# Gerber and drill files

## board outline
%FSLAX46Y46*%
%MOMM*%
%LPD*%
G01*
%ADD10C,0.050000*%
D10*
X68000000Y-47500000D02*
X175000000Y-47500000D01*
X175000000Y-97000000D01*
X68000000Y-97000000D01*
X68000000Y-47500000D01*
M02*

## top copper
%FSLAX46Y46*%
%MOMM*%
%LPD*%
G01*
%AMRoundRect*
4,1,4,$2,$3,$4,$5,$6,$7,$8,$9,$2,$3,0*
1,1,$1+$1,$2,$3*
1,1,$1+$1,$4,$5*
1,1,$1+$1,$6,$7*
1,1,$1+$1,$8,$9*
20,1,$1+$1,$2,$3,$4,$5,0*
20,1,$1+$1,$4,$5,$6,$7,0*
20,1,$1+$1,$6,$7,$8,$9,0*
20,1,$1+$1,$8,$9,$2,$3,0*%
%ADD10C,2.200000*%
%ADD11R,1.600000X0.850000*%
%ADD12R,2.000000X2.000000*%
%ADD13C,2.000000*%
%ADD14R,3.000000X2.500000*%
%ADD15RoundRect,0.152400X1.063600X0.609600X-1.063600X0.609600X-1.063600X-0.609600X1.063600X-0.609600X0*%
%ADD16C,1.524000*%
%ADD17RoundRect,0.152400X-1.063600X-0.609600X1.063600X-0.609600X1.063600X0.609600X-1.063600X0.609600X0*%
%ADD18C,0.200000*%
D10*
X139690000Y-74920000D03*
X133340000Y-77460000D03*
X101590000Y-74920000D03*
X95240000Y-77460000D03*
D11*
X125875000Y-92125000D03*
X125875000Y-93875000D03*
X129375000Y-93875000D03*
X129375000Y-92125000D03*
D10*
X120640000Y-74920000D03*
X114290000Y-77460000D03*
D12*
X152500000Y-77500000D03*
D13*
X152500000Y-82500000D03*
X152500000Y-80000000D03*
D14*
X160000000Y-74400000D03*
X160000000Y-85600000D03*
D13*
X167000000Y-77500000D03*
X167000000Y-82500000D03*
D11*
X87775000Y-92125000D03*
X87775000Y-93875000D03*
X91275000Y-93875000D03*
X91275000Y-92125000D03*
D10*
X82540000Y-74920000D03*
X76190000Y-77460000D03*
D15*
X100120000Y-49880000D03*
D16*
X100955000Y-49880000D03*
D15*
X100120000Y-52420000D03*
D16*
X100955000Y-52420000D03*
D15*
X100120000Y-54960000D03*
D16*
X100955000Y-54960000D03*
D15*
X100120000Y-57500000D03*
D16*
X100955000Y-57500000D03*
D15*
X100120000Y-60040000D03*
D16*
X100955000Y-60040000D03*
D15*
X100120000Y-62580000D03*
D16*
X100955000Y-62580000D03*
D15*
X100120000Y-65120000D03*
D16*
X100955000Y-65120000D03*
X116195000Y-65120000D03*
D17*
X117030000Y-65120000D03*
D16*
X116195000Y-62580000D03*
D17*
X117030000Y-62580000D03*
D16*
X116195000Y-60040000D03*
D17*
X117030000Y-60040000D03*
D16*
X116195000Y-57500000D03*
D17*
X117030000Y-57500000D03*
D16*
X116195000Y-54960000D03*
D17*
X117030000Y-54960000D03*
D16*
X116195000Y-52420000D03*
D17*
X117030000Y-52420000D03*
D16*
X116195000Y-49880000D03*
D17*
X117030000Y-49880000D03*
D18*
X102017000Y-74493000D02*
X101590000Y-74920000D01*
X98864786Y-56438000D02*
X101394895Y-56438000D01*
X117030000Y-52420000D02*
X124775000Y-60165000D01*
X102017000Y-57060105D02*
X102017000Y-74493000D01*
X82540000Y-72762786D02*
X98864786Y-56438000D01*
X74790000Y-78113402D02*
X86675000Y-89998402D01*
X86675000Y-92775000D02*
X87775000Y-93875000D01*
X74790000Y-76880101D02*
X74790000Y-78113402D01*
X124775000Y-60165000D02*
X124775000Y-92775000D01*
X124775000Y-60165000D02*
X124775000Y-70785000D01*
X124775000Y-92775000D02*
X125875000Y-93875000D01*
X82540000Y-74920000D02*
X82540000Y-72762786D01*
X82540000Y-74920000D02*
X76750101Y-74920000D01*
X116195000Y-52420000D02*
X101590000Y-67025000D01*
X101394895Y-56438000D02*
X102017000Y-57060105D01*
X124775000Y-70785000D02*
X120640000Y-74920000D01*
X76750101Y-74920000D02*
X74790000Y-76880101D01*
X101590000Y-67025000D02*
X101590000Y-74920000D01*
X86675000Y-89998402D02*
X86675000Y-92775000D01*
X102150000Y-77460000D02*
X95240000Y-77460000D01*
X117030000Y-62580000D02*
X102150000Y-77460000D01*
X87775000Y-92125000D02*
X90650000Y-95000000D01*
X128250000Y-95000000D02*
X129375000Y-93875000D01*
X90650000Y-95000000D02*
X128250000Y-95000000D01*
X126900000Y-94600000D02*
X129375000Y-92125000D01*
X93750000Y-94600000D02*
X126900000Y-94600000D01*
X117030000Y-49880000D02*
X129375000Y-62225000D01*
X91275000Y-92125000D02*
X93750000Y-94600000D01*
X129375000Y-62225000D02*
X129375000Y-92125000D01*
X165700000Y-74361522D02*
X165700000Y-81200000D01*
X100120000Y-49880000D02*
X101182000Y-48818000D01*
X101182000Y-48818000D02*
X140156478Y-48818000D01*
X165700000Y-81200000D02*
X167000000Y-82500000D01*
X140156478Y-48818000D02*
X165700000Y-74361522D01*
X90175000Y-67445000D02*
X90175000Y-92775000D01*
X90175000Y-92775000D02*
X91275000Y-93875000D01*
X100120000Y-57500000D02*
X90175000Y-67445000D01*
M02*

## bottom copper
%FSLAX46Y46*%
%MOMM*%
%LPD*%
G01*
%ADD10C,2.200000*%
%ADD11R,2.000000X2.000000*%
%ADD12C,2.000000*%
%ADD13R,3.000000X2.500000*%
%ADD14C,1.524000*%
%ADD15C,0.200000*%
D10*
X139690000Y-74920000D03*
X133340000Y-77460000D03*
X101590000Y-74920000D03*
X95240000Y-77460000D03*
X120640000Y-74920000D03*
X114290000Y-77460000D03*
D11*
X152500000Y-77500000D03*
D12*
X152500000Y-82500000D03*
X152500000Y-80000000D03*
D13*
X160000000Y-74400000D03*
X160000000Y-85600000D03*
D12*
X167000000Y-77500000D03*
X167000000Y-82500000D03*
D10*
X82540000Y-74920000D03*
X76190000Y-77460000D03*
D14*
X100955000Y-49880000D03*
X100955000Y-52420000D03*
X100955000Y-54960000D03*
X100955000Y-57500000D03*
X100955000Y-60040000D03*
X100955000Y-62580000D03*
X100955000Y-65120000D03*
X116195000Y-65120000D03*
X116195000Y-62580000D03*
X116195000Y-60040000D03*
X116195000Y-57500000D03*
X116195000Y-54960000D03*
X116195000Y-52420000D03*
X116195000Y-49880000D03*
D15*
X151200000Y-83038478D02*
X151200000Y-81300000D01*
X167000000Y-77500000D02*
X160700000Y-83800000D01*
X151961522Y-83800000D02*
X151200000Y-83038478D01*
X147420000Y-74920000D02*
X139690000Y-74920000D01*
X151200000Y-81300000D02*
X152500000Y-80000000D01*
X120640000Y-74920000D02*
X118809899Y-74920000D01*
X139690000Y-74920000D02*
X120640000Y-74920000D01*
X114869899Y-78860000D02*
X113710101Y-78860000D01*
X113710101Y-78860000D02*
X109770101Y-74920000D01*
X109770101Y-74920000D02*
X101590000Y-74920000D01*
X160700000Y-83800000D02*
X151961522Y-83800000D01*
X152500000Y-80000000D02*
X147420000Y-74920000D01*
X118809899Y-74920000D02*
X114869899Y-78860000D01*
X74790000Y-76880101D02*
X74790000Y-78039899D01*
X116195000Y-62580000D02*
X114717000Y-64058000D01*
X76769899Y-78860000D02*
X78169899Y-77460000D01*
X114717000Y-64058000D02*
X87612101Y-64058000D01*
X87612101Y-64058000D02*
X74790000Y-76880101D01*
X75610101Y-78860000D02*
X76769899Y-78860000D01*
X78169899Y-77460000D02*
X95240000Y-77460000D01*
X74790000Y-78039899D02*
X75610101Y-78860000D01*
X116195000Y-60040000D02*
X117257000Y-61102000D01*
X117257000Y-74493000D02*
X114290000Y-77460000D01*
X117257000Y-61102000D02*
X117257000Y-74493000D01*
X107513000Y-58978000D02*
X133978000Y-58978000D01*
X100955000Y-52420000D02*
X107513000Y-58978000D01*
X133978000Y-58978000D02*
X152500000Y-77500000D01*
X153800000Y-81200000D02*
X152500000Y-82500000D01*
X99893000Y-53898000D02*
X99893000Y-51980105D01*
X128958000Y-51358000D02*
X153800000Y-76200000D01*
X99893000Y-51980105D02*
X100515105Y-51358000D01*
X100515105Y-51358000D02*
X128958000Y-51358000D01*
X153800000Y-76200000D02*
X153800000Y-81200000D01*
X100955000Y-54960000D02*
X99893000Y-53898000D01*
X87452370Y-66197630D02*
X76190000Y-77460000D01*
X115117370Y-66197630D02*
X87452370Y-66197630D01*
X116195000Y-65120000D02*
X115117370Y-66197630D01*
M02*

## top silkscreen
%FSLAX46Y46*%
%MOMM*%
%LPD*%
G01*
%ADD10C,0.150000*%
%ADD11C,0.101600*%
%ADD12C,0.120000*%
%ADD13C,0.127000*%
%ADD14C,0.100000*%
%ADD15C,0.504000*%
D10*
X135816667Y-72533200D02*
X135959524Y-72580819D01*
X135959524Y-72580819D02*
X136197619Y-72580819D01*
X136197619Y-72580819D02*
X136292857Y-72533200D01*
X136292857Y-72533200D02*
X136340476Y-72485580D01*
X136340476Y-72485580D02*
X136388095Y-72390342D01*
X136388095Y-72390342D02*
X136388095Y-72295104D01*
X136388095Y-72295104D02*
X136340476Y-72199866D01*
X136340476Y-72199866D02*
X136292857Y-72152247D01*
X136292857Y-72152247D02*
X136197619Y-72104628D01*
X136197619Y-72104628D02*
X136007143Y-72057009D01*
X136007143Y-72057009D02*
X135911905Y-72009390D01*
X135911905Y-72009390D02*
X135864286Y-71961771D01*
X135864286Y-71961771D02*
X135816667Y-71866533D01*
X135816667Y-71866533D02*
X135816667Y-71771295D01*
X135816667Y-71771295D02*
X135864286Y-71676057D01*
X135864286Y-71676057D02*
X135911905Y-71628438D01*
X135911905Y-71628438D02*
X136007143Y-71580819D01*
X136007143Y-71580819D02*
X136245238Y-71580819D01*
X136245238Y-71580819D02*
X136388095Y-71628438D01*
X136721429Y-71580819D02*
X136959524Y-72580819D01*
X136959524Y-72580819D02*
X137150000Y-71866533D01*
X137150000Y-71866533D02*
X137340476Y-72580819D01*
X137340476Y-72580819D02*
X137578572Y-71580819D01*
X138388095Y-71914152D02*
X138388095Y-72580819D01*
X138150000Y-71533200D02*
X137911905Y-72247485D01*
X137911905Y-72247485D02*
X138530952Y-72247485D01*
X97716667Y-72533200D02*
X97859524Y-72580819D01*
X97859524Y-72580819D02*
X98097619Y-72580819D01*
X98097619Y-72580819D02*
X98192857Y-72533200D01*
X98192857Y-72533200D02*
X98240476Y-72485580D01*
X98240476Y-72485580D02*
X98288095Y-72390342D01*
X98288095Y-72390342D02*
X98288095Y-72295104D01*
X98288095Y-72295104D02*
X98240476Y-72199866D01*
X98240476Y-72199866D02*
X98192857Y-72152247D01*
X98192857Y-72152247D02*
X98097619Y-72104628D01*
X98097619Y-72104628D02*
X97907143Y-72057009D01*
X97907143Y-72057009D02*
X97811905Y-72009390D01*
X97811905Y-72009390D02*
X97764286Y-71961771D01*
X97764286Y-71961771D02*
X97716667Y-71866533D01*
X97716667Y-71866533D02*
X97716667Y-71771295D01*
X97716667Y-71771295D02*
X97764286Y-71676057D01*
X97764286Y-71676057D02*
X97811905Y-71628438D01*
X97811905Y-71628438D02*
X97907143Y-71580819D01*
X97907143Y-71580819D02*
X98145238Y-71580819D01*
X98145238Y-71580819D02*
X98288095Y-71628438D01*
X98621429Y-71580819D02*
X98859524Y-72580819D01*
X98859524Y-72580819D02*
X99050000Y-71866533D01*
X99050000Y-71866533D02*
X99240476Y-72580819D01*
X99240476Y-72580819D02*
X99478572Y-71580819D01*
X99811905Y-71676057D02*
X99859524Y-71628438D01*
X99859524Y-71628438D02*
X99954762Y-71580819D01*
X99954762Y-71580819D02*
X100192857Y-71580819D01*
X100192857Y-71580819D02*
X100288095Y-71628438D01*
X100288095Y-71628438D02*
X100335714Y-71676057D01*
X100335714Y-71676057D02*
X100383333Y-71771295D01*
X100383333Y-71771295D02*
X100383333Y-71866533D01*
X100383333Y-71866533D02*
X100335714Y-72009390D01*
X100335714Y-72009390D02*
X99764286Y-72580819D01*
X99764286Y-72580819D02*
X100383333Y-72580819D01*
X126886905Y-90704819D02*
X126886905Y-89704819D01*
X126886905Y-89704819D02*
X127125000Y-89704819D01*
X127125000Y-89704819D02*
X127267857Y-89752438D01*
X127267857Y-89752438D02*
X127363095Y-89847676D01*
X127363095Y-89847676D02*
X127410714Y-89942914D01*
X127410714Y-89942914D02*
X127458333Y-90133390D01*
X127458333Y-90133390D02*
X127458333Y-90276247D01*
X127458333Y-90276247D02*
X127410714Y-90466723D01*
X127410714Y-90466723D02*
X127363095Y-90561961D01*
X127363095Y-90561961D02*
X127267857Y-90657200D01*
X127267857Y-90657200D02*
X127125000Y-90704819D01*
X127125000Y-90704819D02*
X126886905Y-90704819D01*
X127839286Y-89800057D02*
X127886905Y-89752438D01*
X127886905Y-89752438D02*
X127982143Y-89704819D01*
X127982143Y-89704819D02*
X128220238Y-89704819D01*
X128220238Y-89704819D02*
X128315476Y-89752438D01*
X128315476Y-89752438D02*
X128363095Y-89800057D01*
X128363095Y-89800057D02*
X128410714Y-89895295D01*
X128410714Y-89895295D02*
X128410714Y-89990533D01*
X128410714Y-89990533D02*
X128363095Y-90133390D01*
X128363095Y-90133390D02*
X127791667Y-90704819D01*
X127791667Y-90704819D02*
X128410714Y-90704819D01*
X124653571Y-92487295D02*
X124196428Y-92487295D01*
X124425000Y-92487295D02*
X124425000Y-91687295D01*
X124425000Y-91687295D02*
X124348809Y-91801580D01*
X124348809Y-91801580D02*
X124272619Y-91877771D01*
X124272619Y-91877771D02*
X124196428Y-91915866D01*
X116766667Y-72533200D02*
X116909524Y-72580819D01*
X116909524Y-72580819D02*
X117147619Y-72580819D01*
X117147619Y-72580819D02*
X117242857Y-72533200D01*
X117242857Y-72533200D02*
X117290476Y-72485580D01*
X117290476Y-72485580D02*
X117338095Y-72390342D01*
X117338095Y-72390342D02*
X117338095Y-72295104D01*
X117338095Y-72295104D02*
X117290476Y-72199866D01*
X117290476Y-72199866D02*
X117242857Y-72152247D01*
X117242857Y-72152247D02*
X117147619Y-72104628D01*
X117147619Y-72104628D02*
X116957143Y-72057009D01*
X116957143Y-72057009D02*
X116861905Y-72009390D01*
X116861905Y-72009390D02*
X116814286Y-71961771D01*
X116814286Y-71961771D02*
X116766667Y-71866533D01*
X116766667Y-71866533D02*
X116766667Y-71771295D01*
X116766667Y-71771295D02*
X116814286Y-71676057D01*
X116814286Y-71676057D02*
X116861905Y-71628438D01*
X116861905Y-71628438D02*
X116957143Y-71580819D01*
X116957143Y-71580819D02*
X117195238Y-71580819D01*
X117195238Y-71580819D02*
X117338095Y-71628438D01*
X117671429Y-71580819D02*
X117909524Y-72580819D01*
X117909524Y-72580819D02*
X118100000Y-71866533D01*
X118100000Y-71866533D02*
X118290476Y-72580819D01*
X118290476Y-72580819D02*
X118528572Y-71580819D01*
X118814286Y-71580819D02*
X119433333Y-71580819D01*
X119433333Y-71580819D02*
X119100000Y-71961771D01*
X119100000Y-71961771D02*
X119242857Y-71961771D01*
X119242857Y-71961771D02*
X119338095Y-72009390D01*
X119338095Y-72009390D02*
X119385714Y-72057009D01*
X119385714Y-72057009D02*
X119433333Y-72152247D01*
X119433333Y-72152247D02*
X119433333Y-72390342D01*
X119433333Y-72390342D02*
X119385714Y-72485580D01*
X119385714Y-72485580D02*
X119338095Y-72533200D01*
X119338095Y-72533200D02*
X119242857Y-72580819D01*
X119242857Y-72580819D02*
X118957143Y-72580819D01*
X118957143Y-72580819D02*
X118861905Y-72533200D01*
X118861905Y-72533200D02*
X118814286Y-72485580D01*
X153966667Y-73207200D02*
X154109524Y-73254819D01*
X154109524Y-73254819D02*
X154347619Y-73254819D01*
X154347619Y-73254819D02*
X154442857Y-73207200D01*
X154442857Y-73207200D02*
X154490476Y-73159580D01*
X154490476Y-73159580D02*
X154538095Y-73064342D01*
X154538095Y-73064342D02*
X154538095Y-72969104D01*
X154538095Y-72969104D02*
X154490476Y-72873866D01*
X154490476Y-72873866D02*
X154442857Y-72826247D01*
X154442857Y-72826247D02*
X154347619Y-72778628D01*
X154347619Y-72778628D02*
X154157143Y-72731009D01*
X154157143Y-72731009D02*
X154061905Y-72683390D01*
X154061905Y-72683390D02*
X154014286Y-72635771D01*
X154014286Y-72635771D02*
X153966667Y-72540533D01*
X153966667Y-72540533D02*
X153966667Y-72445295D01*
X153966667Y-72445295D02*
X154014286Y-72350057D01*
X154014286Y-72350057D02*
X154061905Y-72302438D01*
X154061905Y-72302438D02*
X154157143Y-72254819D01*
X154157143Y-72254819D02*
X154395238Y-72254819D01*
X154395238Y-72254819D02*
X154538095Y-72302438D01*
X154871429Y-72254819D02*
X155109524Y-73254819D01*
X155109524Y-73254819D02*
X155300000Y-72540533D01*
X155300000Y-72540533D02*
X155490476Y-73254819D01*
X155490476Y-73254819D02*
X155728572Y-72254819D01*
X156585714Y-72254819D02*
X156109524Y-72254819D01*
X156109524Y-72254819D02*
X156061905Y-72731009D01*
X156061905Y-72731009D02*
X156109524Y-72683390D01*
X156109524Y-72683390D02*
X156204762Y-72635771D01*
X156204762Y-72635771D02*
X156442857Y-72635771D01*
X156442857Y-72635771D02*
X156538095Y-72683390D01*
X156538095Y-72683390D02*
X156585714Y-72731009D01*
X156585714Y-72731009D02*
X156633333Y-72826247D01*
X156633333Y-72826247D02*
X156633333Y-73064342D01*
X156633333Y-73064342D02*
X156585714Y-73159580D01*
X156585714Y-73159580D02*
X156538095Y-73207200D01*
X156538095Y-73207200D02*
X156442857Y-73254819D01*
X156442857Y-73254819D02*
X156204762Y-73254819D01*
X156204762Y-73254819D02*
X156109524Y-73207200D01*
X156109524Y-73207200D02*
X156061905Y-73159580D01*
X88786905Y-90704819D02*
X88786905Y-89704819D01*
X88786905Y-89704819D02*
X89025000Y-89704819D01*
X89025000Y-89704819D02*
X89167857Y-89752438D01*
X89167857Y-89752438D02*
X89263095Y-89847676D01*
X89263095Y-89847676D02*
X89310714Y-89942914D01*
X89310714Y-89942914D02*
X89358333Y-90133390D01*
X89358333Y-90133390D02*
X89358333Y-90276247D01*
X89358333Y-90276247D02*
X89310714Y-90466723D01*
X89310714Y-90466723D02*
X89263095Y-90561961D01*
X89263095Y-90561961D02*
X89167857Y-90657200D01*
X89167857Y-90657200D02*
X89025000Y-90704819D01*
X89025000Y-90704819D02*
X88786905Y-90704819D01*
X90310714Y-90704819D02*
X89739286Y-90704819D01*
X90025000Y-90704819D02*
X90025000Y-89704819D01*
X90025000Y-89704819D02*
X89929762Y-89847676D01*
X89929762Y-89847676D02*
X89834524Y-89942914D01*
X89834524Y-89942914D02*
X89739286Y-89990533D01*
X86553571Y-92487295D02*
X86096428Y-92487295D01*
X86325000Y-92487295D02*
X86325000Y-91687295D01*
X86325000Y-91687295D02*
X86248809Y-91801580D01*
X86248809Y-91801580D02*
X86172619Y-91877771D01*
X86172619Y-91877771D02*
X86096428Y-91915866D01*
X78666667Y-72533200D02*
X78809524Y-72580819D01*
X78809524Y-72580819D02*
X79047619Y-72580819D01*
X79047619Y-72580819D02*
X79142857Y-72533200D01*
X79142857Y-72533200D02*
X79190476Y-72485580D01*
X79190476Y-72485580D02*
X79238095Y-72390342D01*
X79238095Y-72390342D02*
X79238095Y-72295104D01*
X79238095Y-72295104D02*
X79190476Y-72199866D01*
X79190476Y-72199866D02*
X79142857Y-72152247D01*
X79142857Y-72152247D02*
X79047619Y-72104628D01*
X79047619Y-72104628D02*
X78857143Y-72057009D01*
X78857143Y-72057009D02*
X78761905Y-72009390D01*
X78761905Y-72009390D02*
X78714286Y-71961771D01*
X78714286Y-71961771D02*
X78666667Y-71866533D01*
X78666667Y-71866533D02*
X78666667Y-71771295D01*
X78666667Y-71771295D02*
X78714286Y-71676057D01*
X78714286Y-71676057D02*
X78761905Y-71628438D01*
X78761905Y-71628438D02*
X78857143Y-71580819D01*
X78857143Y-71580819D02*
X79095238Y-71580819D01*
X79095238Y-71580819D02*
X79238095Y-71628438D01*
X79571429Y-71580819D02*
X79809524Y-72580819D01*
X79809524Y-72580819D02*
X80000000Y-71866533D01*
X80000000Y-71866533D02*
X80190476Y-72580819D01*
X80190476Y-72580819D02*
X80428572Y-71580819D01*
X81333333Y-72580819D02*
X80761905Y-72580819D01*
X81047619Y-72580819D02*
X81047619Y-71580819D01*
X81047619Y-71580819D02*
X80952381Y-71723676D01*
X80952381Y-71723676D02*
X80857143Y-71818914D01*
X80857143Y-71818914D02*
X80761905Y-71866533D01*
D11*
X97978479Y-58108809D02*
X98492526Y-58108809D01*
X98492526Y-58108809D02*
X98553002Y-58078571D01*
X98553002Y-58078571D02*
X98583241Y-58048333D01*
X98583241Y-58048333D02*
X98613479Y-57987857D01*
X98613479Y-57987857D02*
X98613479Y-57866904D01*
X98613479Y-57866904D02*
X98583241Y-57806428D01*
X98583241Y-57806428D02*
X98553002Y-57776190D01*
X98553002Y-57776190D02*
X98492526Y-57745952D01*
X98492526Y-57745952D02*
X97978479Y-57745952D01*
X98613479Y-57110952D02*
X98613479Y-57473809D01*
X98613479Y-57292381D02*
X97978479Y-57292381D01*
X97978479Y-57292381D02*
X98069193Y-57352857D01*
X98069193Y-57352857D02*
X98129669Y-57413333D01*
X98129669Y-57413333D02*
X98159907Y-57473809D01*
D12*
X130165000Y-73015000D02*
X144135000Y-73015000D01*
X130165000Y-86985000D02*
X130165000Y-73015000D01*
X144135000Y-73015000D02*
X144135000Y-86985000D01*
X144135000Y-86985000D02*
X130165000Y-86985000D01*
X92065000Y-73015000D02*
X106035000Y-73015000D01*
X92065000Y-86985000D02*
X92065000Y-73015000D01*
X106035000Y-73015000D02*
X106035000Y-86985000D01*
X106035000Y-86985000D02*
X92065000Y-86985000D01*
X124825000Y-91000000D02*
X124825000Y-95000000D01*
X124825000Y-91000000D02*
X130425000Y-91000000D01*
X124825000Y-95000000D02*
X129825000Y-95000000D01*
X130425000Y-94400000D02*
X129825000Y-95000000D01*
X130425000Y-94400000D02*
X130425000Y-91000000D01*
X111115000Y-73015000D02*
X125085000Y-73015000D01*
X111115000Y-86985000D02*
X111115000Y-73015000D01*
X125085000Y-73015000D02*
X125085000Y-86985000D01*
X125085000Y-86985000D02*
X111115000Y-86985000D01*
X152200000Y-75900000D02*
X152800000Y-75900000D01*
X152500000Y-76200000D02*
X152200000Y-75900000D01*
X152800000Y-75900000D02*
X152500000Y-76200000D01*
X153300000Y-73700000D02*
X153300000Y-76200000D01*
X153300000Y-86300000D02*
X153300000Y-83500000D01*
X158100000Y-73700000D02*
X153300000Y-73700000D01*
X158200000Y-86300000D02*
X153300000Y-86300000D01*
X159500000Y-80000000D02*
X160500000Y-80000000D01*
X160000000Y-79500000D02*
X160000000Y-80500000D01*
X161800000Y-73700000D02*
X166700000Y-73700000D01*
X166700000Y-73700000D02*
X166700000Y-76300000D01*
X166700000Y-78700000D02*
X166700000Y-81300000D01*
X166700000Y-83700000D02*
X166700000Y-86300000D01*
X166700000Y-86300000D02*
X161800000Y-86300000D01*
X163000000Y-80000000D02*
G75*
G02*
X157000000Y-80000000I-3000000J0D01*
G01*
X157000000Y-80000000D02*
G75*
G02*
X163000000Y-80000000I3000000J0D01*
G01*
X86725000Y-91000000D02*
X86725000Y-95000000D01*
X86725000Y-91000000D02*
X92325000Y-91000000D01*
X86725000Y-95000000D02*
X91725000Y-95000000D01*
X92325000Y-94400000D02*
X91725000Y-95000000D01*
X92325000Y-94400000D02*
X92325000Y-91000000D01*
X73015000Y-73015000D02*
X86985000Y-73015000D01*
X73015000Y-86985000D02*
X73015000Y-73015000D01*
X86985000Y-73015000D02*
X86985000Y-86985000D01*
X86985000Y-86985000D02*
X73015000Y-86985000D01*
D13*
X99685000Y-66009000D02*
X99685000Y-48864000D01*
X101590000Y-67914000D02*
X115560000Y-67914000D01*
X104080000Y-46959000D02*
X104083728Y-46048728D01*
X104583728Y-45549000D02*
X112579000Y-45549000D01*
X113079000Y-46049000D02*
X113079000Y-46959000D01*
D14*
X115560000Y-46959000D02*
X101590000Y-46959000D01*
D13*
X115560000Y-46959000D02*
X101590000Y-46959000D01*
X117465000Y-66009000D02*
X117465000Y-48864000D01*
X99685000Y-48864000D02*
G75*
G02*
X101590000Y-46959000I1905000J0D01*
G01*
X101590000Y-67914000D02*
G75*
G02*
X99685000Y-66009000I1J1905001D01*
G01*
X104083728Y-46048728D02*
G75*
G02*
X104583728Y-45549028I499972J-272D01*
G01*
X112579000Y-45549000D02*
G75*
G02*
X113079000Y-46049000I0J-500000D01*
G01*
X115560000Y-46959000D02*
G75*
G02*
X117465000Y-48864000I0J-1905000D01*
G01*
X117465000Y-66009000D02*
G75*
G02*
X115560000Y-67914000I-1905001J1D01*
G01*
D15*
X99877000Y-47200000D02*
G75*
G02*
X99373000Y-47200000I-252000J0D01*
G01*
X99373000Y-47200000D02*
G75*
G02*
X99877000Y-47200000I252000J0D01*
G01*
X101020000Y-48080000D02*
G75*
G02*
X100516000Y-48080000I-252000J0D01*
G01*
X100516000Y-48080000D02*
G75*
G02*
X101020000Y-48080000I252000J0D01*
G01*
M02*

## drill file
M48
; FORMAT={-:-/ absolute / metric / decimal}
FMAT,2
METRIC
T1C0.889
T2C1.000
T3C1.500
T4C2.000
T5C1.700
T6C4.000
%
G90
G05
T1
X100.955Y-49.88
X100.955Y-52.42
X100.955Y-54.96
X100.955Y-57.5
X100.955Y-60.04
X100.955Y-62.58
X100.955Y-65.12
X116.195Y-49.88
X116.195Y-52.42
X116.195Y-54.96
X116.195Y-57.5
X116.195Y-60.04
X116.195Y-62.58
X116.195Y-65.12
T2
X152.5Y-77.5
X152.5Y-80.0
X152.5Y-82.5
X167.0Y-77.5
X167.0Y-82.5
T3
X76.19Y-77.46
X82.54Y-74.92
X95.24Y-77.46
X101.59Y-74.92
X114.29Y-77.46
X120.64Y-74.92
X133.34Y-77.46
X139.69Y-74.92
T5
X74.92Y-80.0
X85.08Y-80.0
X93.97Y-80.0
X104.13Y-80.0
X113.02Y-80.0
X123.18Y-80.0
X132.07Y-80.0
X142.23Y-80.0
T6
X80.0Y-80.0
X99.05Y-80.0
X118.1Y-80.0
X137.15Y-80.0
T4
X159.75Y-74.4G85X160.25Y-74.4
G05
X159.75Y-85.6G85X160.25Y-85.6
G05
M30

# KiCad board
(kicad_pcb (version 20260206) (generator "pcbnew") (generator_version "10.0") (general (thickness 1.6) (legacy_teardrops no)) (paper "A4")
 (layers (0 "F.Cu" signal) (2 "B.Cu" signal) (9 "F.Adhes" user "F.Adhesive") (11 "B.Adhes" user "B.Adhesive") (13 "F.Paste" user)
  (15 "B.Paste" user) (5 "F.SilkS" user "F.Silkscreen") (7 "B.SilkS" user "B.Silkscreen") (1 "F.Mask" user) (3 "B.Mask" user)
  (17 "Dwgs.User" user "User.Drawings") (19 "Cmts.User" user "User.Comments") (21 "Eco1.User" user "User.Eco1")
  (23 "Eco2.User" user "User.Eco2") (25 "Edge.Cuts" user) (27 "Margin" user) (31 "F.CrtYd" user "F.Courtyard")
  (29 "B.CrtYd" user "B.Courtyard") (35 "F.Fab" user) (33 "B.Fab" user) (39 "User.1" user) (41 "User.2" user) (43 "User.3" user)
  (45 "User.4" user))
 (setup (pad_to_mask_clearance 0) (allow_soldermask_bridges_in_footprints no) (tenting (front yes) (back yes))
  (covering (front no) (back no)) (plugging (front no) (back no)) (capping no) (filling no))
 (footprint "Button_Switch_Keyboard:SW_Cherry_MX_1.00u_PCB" (layer "F.Cu") (at 139.69 74.92)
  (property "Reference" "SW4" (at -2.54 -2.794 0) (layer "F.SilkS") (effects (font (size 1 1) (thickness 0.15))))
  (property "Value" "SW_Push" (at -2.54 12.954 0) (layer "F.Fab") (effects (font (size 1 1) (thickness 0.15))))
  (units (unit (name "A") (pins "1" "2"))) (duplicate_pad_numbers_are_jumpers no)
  (fp_line (start -9.525 -1.905) (end 4.445 -1.905) (stroke (width 0.12) (type solid)) (layer "F.SilkS"))
  (fp_line (start -9.525 12.065) (end -9.525 -1.905) (stroke (width 0.12) (type solid)) (layer "F.SilkS"))
  (fp_line (start 4.445 -1.905) (end 4.445 12.065) (stroke (width 0.12) (type solid)) (layer "F.SilkS"))
  (fp_line (start 4.445 12.065) (end -9.525 12.065) (stroke (width 0.12) (type solid)) (layer "F.SilkS"))
  (pad "" np_thru_hole circle (at -7.62 5.08) (size 1.7 1.7) (drill 1.7) (layers "*.Cu" "*.Mask"))
  (pad "" np_thru_hole circle (at -2.54 5.08) (size 4 4) (drill 4) (layers "*.Cu" "*.Mask"))
  (pad "" np_thru_hole circle (at 2.54 5.08) (size 1.7 1.7) (drill 1.7) (layers "*.Cu" "*.Mask"))
  (pad "1" thru_hole circle (at 0 0) (size 2.2 2.2) (drill 1.5) (layers "*.Cu" "*.Mask") (remove_unused_layers no) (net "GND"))
  (pad "2" thru_hole circle (at -6.35 2.54) (size 2.2 2.2) (drill 1.5) (layers "*.Cu" "*.Mask") (remove_unused_layers no)
   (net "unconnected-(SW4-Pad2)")))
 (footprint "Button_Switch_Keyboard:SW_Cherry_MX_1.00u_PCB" (layer "F.Cu") (at 101.59 74.92)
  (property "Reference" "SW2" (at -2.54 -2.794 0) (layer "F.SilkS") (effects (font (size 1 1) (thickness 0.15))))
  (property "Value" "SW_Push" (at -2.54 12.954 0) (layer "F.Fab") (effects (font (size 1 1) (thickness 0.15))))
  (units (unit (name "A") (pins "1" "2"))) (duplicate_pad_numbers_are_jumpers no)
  (fp_line (start -9.525 -1.905) (end 4.445 -1.905) (stroke (width 0.12) (type solid)) (layer "F.SilkS"))
  (fp_line (start -9.525 12.065) (end -9.525 -1.905) (stroke (width 0.12) (type solid)) (layer "F.SilkS"))
  (fp_line (start 4.445 -1.905) (end 4.445 12.065) (stroke (width 0.12) (type solid)) (layer "F.SilkS"))
  (fp_line (start 4.445 12.065) (end -9.525 12.065) (stroke (width 0.12) (type solid)) (layer "F.SilkS"))
  (pad "" np_thru_hole circle (at -7.62 5.08) (size 1.7 1.7) (drill 1.7) (layers "*.Cu" "*.Mask"))
  (pad "" np_thru_hole circle (at -2.54 5.08) (size 4 4) (drill 4) (layers "*.Cu" "*.Mask"))
  (pad "" np_thru_hole circle (at 2.54 5.08) (size 1.7 1.7) (drill 1.7) (layers "*.Cu" "*.Mask"))
  (pad "1" thru_hole circle (at 0 0) (size 2.2 2.2) (drill 1.5) (layers "*.Cu" "*.Mask") (remove_unused_layers no) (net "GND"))
  (pad "2" thru_hole circle (at -6.35 2.54) (size 2.2 2.2) (drill 1.5) (layers "*.Cu" "*.Mask") (remove_unused_layers no)
   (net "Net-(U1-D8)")))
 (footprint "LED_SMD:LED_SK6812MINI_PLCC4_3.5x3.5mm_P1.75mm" (layer "F.Cu") (at 127.625 93)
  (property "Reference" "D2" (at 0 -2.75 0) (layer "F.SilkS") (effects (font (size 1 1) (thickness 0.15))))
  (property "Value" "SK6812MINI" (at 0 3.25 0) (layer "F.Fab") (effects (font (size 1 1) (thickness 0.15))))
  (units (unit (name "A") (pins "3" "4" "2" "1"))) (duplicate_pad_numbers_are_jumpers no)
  (fp_line (start -2.8 -2) (end -2.8 2) (stroke (width 0.12) (type default)) (layer "F.SilkS"))
  (fp_line (start -2.8 -2) (end 2.8 -2) (stroke (width 0.12) (type solid)) (layer "F.SilkS"))
  (fp_line (start -2.8 2) (end 2.2 2) (stroke (width 0.12) (type solid)) (layer "F.SilkS"))
  (fp_line (start 2.8 1.4) (end 2.2 2) (stroke (width 0.12) (type default)) (layer "F.SilkS"))
  (fp_line (start 2.8 1.4) (end 2.8 -2) (stroke (width 0.12) (type solid)) (layer "F.SilkS"))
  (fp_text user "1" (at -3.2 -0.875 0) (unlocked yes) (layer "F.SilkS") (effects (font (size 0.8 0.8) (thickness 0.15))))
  (pad "1" smd rect (at -1.75 -0.875) (size 1.6 0.85) (layers "F.Cu" "F.Mask" "F.Paste") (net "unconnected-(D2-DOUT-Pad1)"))
  (pad "2" smd rect (at -1.75 0.875) (size 1.6 0.85) (layers "F.Cu" "F.Mask" "F.Paste") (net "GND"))
  (pad "3" smd rect (at 1.75 0.875) (size 1.6 0.85) (layers "F.Cu" "F.Mask" "F.Paste") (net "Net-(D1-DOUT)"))
  (pad "4" smd rect (at 1.75 -0.875) (size 1.6 0.85) (layers "F.Cu" "F.Mask" "F.Paste") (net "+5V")))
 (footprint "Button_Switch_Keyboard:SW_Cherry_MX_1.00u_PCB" (layer "F.Cu") (at 120.64 74.92)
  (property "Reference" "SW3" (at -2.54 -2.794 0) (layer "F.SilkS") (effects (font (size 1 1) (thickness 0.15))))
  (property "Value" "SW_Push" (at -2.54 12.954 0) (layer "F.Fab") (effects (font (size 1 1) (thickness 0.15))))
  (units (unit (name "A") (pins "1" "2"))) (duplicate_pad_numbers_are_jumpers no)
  (fp_line (start -9.525 -1.905) (end 4.445 -1.905) (stroke (width 0.12) (type solid)) (layer "F.SilkS"))
  (fp_line (start -9.525 12.065) (end -9.525 -1.905) (stroke (width 0.12) (type solid)) (layer "F.SilkS"))
  (fp_line (start 4.445 -1.905) (end 4.445 12.065) (stroke (width 0.12) (type solid)) (layer "F.SilkS"))
  (fp_line (start 4.445 12.065) (end -9.525 12.065) (stroke (width 0.12) (type solid)) (layer "F.SilkS"))
  (pad "" np_thru_hole circle (at -7.62 5.08) (size 1.7 1.7) (drill 1.7) (layers "*.Cu" "*.Mask"))
  (pad "" np_thru_hole circle (at -2.54 5.08) (size 4 4) (drill 4) (layers "*.Cu" "*.Mask"))
  (pad "" np_thru_hole circle (at 2.54 5.08) (size 1.7 1.7) (drill 1.7) (layers "*.Cu" "*.Mask"))
  (pad "1" thru_hole circle (at 0 0) (size 2.2 2.2) (drill 1.5) (layers "*.Cu" "*.Mask") (remove_unused_layers no) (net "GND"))
  (pad "2" thru_hole circle (at -6.35 2.54) (size 2.2 2.2) (drill 1.5) (layers "*.Cu" "*.Mask") (remove_unused_layers no)
   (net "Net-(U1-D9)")))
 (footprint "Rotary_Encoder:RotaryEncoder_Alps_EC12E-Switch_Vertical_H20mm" (layer "F.Cu") (at 152.5 77.5)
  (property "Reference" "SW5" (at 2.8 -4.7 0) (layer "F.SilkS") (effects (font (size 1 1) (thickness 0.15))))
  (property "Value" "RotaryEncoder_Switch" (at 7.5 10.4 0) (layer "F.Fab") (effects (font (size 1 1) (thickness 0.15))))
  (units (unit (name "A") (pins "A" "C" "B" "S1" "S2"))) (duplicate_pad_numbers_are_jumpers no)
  (fp_line (start -0.3 -1.6) (end 0.3 -1.6) (stroke (width 0.12) (type solid)) (layer "F.SilkS"))
  (fp_line (start 0 -1.3) (end -0.3 -1.6) (stroke (width 0.12) (type solid)) (layer "F.SilkS"))
  (fp_line (start 0.3 -1.6) (end 0 -1.3) (stroke (width 0.12) (type solid)) (layer "F.SilkS"))
  (fp_line (start 0.8 -3.8) (end 0.8 -1.3) (stroke (width 0.12) (type solid)) (layer "F.SilkS"))
  (fp_line (start 0.8 8.8) (end 0.8 6) (stroke (width 0.12) (type solid)) (layer "F.SilkS"))
  (fp_line (start 5.6 -3.8) (end 0.8 -3.8) (stroke (width 0.12) (type solid)) (layer "F.SilkS"))
  (fp_line (start 5.7 8.8) (end 0.8 8.8) (stroke (width 0.12) (type solid)) (layer "F.SilkS"))
  (fp_line (start 7 2.5) (end 8 2.5) (stroke (width 0.12) (type solid)) (layer "F.SilkS"))
  (fp_line (start 7.5 2) (end 7.5 3) (stroke (width 0.12) (type solid)) (layer "F.SilkS"))
  (fp_line (start 9.3 -3.8) (end 14.2 -3.8) (stroke (width 0.12) (type solid)) (layer "F.SilkS"))
  (fp_line (start 14.2 -3.8) (end 14.2 -1.2) (stroke (width 0.12) (type solid)) (layer "F.SilkS"))
  (fp_line (start 14.2 1.2) (end 14.2 3.8) (stroke (width 0.12) (type solid)) (layer "F.SilkS"))
  (fp_line (start 14.2 6.2) (end 14.2 8.8) (stroke (width 0.12) (type solid)) (layer "F.SilkS"))
  (fp_line (start 14.2 8.8) (end 9.3 8.8) (stroke (width 0.12) (type solid)) (layer "F.SilkS"))
  (fp_circle (center 7.5 2.5) (end 10.5 2.5) (stroke (width 0.12) (type solid)) (fill no) (layer "F.SilkS"))
  (pad "A" thru_hole rect (at 0 0) (size 2 2) (drill 1) (layers "*.Cu" "*.Mask") (remove_unused_layers no) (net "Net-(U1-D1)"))
  (pad "B" thru_hole circle (at 0 5) (size 2 2) (drill 1) (layers "*.Cu" "*.Mask") (remove_unused_layers no) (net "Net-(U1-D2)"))
  (pad "C" thru_hole circle (at 0 2.5) (size 2 2) (drill 1) (layers "*.Cu" "*.Mask") (remove_unused_layers no) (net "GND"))
  (pad "MP" thru_hole rect (at 7.5 -3.1) (size 3 2.5) (drill oval 2.5 2) (layers "*.Cu" "*.Mask") (remove_unused_layers no))
  (pad "MP" thru_hole rect (at 7.5 8.1) (size 3 2.5) (drill oval 2.5 2) (layers "*.Cu" "*.Mask") (remove_unused_layers no))
  (pad "S1" thru_hole circle (at 14.5 0) (size 2 2) (drill 1) (layers "*.Cu" "*.Mask") (remove_unused_layers no) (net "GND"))
  (pad "S2" thru_hole circle (at 14.5 5) (size 2 2) (drill 1) (layers "*.Cu" "*.Mask") (remove_unused_layers no) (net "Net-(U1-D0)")))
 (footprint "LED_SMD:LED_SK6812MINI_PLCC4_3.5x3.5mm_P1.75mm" (layer "F.Cu") (at 89.525 93)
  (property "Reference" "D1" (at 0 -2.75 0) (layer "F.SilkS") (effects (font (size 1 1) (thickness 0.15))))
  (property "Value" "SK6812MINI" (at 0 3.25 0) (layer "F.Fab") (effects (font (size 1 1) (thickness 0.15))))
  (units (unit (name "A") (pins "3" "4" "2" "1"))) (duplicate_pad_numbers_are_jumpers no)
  (fp_line (start -2.8 -2) (end -2.8 2) (stroke (width 0.12) (type default)) (layer "F.SilkS"))
  (fp_line (start -2.8 -2) (end 2.8 -2) (stroke (width 0.12) (type solid)) (layer "F.SilkS"))
  (fp_line (start -2.8 2) (end 2.2 2) (stroke (width 0.12) (type solid)) (layer "F.SilkS"))
  (fp_line (start 2.8 1.4) (end 2.2 2) (stroke (width 0.12) (type default)) (layer "F.SilkS"))
  (fp_line (start 2.8 1.4) (end 2.8 -2) (stroke (width 0.12) (type solid)) (layer "F.SilkS"))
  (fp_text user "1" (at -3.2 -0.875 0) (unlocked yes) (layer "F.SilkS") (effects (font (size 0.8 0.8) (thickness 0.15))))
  (pad "1" smd rect (at -1.75 -0.875) (size 1.6 0.85) (layers "F.Cu" "F.Mask" "F.Paste") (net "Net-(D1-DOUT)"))
  (pad "2" smd rect (at -1.75 0.875) (size 1.6 0.85) (layers "F.Cu" "F.Mask" "F.Paste") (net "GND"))
  (pad "3" smd rect (at 1.75 0.875) (size 1.6 0.85) (layers "F.Cu" "F.Mask" "F.Paste") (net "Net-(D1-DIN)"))
  (pad "4" smd rect (at 1.75 -0.875) (size 1.6 0.85) (layers "F.Cu" "F.Mask" "F.Paste") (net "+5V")))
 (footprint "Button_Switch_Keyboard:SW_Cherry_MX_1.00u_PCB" (layer "F.Cu") (at 82.54 74.92)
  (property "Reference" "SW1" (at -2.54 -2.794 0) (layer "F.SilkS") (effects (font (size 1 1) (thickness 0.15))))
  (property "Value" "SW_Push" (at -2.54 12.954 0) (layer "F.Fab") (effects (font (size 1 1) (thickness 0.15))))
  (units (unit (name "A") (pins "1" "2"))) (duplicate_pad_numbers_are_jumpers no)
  (fp_line (start -9.525 -1.905) (end 4.445 -1.905) (stroke (width 0.12) (type solid)) (layer "F.SilkS"))
  (fp_line (start -9.525 12.065) (end -9.525 -1.905) (stroke (width 0.12) (type solid)) (layer "F.SilkS"))
  (fp_line (start 4.445 -1.905) (end 4.445 12.065) (stroke (width 0.12) (type solid)) (layer "F.SilkS"))
  (fp_line (start 4.445 12.065) (end -9.525 12.065) (stroke (width 0.12) (type solid)) (layer "F.SilkS"))
  (pad "" np_thru_hole circle (at -7.62 5.08) (size 1.7 1.7) (drill 1.7) (layers "*.Cu" "*.Mask"))
  (pad "" np_thru_hole circle (at -2.54 5.08) (size 4 4) (drill 4) (layers "*.Cu" "*.Mask"))
  (pad "" np_thru_hole circle (at 2.54 5.08) (size 1.7 1.7) (drill 1.7) (layers "*.Cu" "*.Mask"))
  (pad "1" thru_hole circle (at 0 0) (size 2.2 2.2) (drill 1.5) (layers "*.Cu" "*.Mask") (remove_unused_layers no) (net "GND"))
  (pad "2" thru_hole circle (at -6.35 2.54) (size 2.2 2.2) (drill 1.5) (layers "*.Cu" "*.Mask") (remove_unused_layers no)
   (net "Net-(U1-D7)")))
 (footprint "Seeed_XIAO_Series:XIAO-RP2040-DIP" (layer "F.Cu") (at 108.575 57.5 90)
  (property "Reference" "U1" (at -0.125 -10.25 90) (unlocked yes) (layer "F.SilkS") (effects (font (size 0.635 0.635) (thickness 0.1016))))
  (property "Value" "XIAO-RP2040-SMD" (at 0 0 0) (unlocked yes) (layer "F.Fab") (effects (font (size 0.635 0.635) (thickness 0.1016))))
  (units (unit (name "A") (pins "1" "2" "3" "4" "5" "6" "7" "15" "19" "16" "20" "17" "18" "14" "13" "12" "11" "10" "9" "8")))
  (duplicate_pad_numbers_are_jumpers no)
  (fp_line (start -8.509 -8.89) (end 8.636 -8.89) (stroke (width 0.127) (type solid)) (layer "F.SilkS"))
  (fp_line (start -10.414 -6.985) (end -10.414 6.985) (stroke (width 0.127) (type solid)) (layer "F.SilkS"))
  (fp_line (start 10.541 -4.495) (end 11.451272 -4.491272) (stroke (width 0.127) (type solid)) (layer "F.SilkS"))
  (fp_line (start 11.951 -3.991272) (end 11.951 4.004) (stroke (width 0.127) (type solid)) (layer "F.SilkS"))
  (fp_line (start 11.451 4.504) (end 10.541 4.504) (stroke (width 0.127) (type solid)) (layer "F.SilkS"))
  (fp_line (start 10.541 6.985) (end 10.541 -6.985) (stroke (width 0.1) (type solid)) (layer "F.SilkS"))
  (fp_line (start 10.541 6.985) (end 10.541 -6.985) (stroke (width 0.127) (type solid)) (layer "F.SilkS"))
  (fp_line (start -8.509 8.89) (end 8.636 8.89) (stroke (width 0.127) (type solid)) (layer "F.SilkS"))
  (fp_arc (start 8.636 -8.89) (mid 9.983038 -8.332038) (end 10.541 -6.985) (stroke (width 0.127) (type solid)) (layer "F.SilkS"))
  (fp_arc (start -10.414 -6.985) (mid -9.856038 -8.332038) (end -8.509 -8.89) (stroke (width 0.127) (type solid)) (layer "F.SilkS"))
  (fp_arc (start 11.451272 -4.491272) (mid 11.804644 -4.344724) (end 11.951 -3.991272) (stroke (width 0.127) (type default))
   (layer "F.SilkS"))
  (fp_arc (start 11.951 4.004) (mid 11.804553 4.357553) (end 11.451 4.504) (stroke (width 0.127) (type default)) (layer "F.SilkS"))
  (fp_arc (start 10.541 6.985) (mid 9.983038 8.332038) (end 8.636 8.89) (stroke (width 0.127) (type solid)) (layer "F.SilkS"))
  (fp_arc (start -8.509 8.89) (mid -9.856038 8.332038) (end -10.414 6.985) (stroke (width 0.127) (type solid)) (layer "F.SilkS"))
  (fp_circle (center 10.3 -8.95) (end 10.554 -8.95) (stroke (width 0.5) (type solid)) (fill yes) (layer "F.SilkS"))
  (fp_circle (center 9.42 -7.807) (end 9.674 -7.807) (stroke (width 0.5) (type solid)) (fill yes) (layer "F.SilkS"))
  (pad "1" smd roundrect (at 7.62 -8.455 180) (size 2.432 1.524) (layers "F.Cu" "F.Mask") (roundrect_rratio 0.1) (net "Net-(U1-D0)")
   (thermal_bridge_angle 45))
  (pad "1" thru_hole circle (at 7.62 -7.62 180) (size 1.524 1.524) (drill 0.889) (layers "*.Cu" "*.Mask") (remove_unused_layers no)
   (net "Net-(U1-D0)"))
  (pad "2" smd roundrect (at 5.08 -8.455 180) (size 2.432 1.524) (layers "F.Cu" "F.Mask") (roundrect_rratio 0.1) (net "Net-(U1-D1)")
   (thermal_bridge_angle 45))
  (pad "2" thru_hole circle (at 5.08 -7.62 180) (size 1.524 1.524) (drill 0.889) (layers "*.Cu" "*.Mask") (remove_unused_layers no)
   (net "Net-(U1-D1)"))
  (pad "3" smd roundrect (at 2.54 -8.455 180) (size 2.432 1.524) (layers "F.Cu" "F.Mask") (roundrect_rratio 0.1) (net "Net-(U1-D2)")
   (thermal_bridge_angle 45))
  (pad "3" thru_hole circle (at 2.54 -7.62 180) (size 1.524 1.524) (drill 0.889) (layers "*.Cu" "*.Mask") (remove_unused_layers no)
   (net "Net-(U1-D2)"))
  (pad "4" smd roundrect (at 0 -8.455 180) (size 2.432 1.524) (layers "F.Cu" "F.Mask") (roundrect_rratio 0.1) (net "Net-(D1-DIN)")
   (thermal_bridge_angle 45))
  (pad "4" thru_hole circle (at 0 -7.62 180) (size 1.524 1.524) (drill 0.889) (layers "*.Cu" "*.Mask") (remove_unused_layers no)
   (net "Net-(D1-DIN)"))
  (pad "5" smd roundrect (at -2.54 -8.455 180) (size 2.432 1.524) (layers "F.Cu" "F.Mask") (roundrect_rratio 0.1)
   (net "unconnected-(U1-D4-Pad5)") (thermal_bridge_angle 45))
  (pad "5" thru_hole circle (at -2.54 -7.62 180) (size 1.524 1.524) (drill 0.889) (layers "*.Cu" "*.Mask") (remove_unused_layers no)
   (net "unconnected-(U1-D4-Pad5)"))
  (pad "6" smd roundrect (at -5.08 -8.455 180) (size 2.432 1.524) (layers "F.Cu" "F.Mask") (roundrect_rratio 0.1)
   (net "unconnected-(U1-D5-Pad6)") (thermal_bridge_angle 45))
  (pad "6" thru_hole circle (at -5.08 -7.62 180) (size 1.524 1.524) (drill 0.889) (layers "*.Cu" "*.Mask") (remove_unused_layers no)
   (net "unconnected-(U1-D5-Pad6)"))
  (pad "7" smd roundrect (at -7.62 -8.455 180) (size 2.432 1.524) (layers "F.Cu" "F.Mask") (roundrect_rratio 0.1)
   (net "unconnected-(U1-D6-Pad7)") (thermal_bridge_angle 45))
  (pad "7" thru_hole circle (at -7.62 -7.62 180) (size 1.524 1.524) (drill 0.889) (layers "*.Cu" "*.Mask") (remove_unused_layers no)
   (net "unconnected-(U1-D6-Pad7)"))
  (pad "8" thru_hole circle (at -7.62 7.62) (size 1.524 1.524) (drill 0.889) (layers "*.Cu" "*.Mask") (remove_unused_layers no)
   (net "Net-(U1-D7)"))
  (pad "8" smd roundrect (at -7.62 8.455) (size 2.432 1.524) (layers "F.Cu" "F.Mask") (roundrect_rratio 0.1) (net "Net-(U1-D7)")
   (thermal_bridge_angle 45))
  (pad "9" thru_hole circle (at -5.08 7.62) (size 1.524 1.524) (drill 0.889) (layers "*.Cu" "*.Mask") (remove_unused_layers no)
   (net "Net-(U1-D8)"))
  (pad "9" smd roundrect (at -5.08 8.455) (size 2.432 1.524) (layers "F.Cu" "F.Mask") (roundrect_rratio 0.1) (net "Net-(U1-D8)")
   (thermal_bridge_angle 45))
  (pad "10" thru_hole circle (at -2.54 7.62) (size 1.524 1.524) (drill 0.889) (layers "*.Cu" "*.Mask") (remove_unused_layers no)
   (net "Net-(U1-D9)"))
  (pad "10" smd roundrect (at -2.54 8.455) (size 2.432 1.524) (layers "F.Cu" "F.Mask") (roundrect_rratio 0.1) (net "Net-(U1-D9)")
   (thermal_bridge_angle 45))
  (pad "11" thru_hole circle (at 0 7.62) (size 1.524 1.524) (drill 0.889) (layers "*.Cu" "*.Mask") (remove_unused_layers no)
   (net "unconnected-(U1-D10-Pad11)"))
  (pad "11" smd roundrect (at 0 8.455) (size 2.432 1.524) (layers "F.Cu" "F.Mask") (roundrect_rratio 0.1) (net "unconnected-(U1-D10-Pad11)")
   (thermal_bridge_angle 45))
  (pad "12" thru_hole circle (at 2.54 7.62) (size 1.524 1.524) (drill 0.889) (layers "*.Cu" "*.Mask") (remove_unused_layers no)
   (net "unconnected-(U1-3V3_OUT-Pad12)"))
  (pad "12" smd roundrect (at 2.54 8.455) (size 2.432 1.524) (layers "F.Cu" "F.Mask") (roundrect_rratio 0.1)
   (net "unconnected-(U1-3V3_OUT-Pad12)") (thermal_bridge_angle 45))
  (pad "13" thru_hole circle (at 5.08 7.62) (size 1.524 1.524) (drill 0.889) (layers "*.Cu" "*.Mask") (remove_unused_layers no) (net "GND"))
  (pad "13" smd roundrect (at 5.08 8.455) (size 2.432 1.524) (layers "F.Cu" "F.Mask") (roundrect_rratio 0.1) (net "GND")
   (thermal_bridge_angle 45))
  (pad "14" thru_hole circle (at 7.62 7.62) (size 1.524 1.524) (drill 0.889) (layers "*.Cu" "*.Mask") (remove_unused_layers no) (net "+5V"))
  (pad "14" smd roundrect (at 7.62 8.455) (size 2.432 1.524) (layers "F.Cu" "F.Mask") (roundrect_rratio 0.1) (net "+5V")
   (thermal_bridge_angle 45)))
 (gr_rect (start 68 47.5) (end 175 97) (stroke (width 0.05) (type default)) (fill no) (layer "Edge.Cuts"))
 (segment (start 102.017 74.493) (end 101.59 74.92) (width 0.2) (layer "F.Cu") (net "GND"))
 (segment (start 98.864786 56.438) (end 101.394895 56.438) (width 0.2) (layer "F.Cu") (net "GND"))
 (segment (start 117.03 52.42) (end 124.775 60.165) (width 0.2) (layer "F.Cu") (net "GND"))
 (segment (start 102.017 57.060105) (end 102.017 74.493) (width 0.2) (layer "F.Cu") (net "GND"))
 (segment (start 82.54 72.762786) (end 98.864786 56.438) (width 0.2) (layer "F.Cu") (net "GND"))
 (segment (start 74.79 78.113402) (end 86.675 89.998402) (width 0.2) (layer "F.Cu") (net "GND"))
 (segment (start 86.675 92.775) (end 87.775 93.875) (width 0.2) (layer "F.Cu") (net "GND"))
 (segment (start 74.79 76.880101) (end 74.79 78.113402) (width 0.2) (layer "F.Cu") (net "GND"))
 (segment (start 124.775 60.165) (end 124.775 92.775) (width 0.2) (layer "F.Cu") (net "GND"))
 (segment (start 124.775 60.165) (end 124.775 70.785) (width 0.2) (layer "F.Cu") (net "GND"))
 (segment (start 124.775 92.775) (end 125.875 93.875) (width 0.2) (layer "F.Cu") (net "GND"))
 (segment (start 82.54 74.92) (end 82.54 72.762786) (width 0.2) (layer "F.Cu") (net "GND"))
 (segment (start 82.54 74.92) (end 76.750101 74.92) (width 0.2) (layer "F.Cu") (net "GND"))
 (segment (start 116.195 52.42) (end 101.59 67.025) (width 0.2) (layer "F.Cu") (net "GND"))
 (segment (start 101.394895 56.438) (end 102.017 57.060105) (width 0.2) (layer "F.Cu") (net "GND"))
 (segment (start 124.775 70.785) (end 120.64 74.92) (width 0.2) (layer "F.Cu") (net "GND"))
 (segment (start 76.750101 74.92) (end 74.79 76.880101) (width 0.2) (layer "F.Cu") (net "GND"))
 (segment (start 101.59 67.025) (end 101.59 74.92) (width 0.2) (layer "F.Cu") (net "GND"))
 (segment (start 86.675 89.998402) (end 86.675 92.775) (width 0.2) (layer "F.Cu") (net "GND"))
 (segment (start 151.2 83.038478) (end 151.2 81.3) (width 0.2) (layer "B.Cu") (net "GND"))
 (segment (start 167 77.5) (end 160.7 83.8) (width 0.2) (layer "B.Cu") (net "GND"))
 (segment (start 151.961522 83.8) (end 151.2 83.038478) (width 0.2) (layer "B.Cu") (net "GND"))
 (segment (start 147.42 74.92) (end 139.69 74.92) (width 0.2) (layer "B.Cu") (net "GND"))
 (segment (start 151.2 81.3) (end 152.5 80) (width 0.2) (layer "B.Cu") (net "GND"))
 (segment (start 120.64 74.92) (end 118.809899 74.92) (width 0.2) (layer "B.Cu") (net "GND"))
 (segment (start 139.69 74.92) (end 120.64 74.92) (width 0.2) (layer "B.Cu") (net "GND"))
 (segment (start 114.869899 78.86) (end 113.710101 78.86) (width 0.2) (layer "B.Cu") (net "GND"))
 (segment (start 113.710101 78.86) (end 109.770101 74.92) (width 0.2) (layer "B.Cu") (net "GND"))
 (segment (start 109.770101 74.92) (end 101.59 74.92) (width 0.2) (layer "B.Cu") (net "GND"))
 (segment (start 160.7 83.8) (end 151.961522 83.8) (width 0.2) (layer "B.Cu") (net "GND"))
 (segment (start 152.5 80) (end 147.42 74.92) (width 0.2) (layer "B.Cu") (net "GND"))
 (segment (start 118.809899 74.92) (end 114.869899 78.86) (width 0.2) (layer "B.Cu") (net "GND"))
 (segment (start 102.15 77.46) (end 95.24 77.46) (width 0.2) (layer "F.Cu") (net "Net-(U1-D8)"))
 (segment (start 117.03 62.58) (end 102.15 77.46) (width 0.2) (layer "F.Cu") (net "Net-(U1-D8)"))
 (segment (start 74.79 76.880101) (end 74.79 78.039899) (width 0.2) (layer "B.Cu") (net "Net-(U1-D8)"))
 (segment (start 116.195 62.58) (end 114.717 64.058) (width 0.2) (layer "B.Cu") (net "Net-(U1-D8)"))
 (segment (start 76.769899 78.86) (end 78.169899 77.46) (width 0.2) (layer "B.Cu") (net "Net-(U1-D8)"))
 (segment (start 114.717 64.058) (end 87.612101 64.058) (width 0.2) (layer "B.Cu") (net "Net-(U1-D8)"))
 (segment (start 87.612101 64.058) (end 74.79 76.880101) (width 0.2) (layer "B.Cu") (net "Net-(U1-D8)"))
 (segment (start 75.610101 78.86) (end 76.769899 78.86) (width 0.2) (layer "B.Cu") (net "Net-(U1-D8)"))
 (segment (start 78.169899 77.46) (end 95.24 77.46) (width 0.2) (layer "B.Cu") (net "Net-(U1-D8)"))
 (segment (start 74.79 78.039899) (end 75.610101 78.86) (width 0.2) (layer "B.Cu") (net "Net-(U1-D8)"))
 (segment (start 87.775 92.125) (end 90.65 95) (width 0.2) (layer "F.Cu") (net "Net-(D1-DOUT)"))
 (segment (start 128.25 95) (end 129.375 93.875) (width 0.2) (layer "F.Cu") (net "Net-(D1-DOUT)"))
 (segment (start 90.65 95) (end 128.25 95) (width 0.2) (layer "F.Cu") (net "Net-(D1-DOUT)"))
 (segment (start 126.9 94.6) (end 129.375 92.125) (width 0.2) (layer "F.Cu") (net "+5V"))
 (segment (start 93.75 94.6) (end 126.9 94.6) (width 0.2) (layer "F.Cu") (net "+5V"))
 (segment (start 117.03 49.88) (end 129.375 62.225) (width 0.2) (layer "F.Cu") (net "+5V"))
 (segment (start 91.275 92.125) (end 93.75 94.6) (width 0.2) (layer "F.Cu") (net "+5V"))
 (segment (start 129.375 62.225) (end 129.375 92.125) (width 0.2) (layer "F.Cu") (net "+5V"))
 (segment (start 116.195 60.04) (end 117.257 61.102) (width 0.2) (layer "B.Cu") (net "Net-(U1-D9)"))
 (segment (start 117.257 74.493) (end 114.29 77.46) (width 0.2) (layer "B.Cu") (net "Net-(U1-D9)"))
 (segment (start 117.257 61.102) (end 117.257 74.493) (width 0.2) (layer "B.Cu") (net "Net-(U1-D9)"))
 (segment (start 107.513 58.978) (end 133.978 58.978) (width 0.2) (layer "B.Cu") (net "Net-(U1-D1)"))
 (segment (start 100.955 52.42) (end 107.513 58.978) (width 0.2) (layer "B.Cu") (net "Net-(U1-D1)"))
 (segment (start 133.978 58.978) (end 152.5 77.5) (width 0.2) (layer "B.Cu") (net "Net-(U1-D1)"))
 (segment (start 153.8 81.2) (end 152.5 82.5) (width 0.2) (layer "B.Cu") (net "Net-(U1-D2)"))
 (segment (start 99.893 53.898) (end 99.893 51.980105) (width 0.2) (layer "B.Cu") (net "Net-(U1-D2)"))
 (segment (start 128.958 51.358) (end 153.8 76.2) (width 0.2) (layer "B.Cu") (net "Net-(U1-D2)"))
 (segment (start 99.893 51.980105) (end 100.515105 51.358) (width 0.2) (layer "B.Cu") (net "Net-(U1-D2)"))
 (segment (start 100.515105 51.358) (end 128.958 51.358) (width 0.2) (layer "B.Cu") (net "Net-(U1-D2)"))
 (segment (start 153.8 76.2) (end 153.8 81.2) (width 0.2) (layer "B.Cu") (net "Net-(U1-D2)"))
 (segment (start 100.955 54.96) (end 99.893 53.898) (width 0.2) (layer "B.Cu") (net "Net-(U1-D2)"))
 (segment (start 165.7 74.361522) (end 165.7 81.2) (width 0.2) (layer "F.Cu") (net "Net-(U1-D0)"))
 (segment (start 100.12 49.88) (end 101.182 48.818) (width 0.2) (layer "F.Cu") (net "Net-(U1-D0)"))
 (segment (start 101.182 48.818) (end 140.156478 48.818) (width 0.2) (layer "F.Cu") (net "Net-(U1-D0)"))
 (segment (start 165.7 81.2) (end 167 82.5) (width 0.2) (layer "F.Cu") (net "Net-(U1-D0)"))
 (segment (start 140.156478 48.818) (end 165.7 74.361522) (width 0.2) (layer "F.Cu") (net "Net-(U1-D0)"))
 (segment (start 90.175 67.445) (end 90.175 92.775) (width 0.2) (layer "F.Cu") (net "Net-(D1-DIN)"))
 (segment (start 90.175 92.775) (end 91.275 93.875) (width 0.2) (layer "F.Cu") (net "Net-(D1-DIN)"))
 (segment (start 100.12 57.5) (end 90.175 67.445) (width 0.2) (layer "F.Cu") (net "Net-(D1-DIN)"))
 (segment (start 87.45237 66.19763) (end 76.19 77.46) (width 0.2) (layer "B.Cu") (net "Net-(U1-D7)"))
 (segment (start 115.11737 66.19763) (end 87.45237 66.19763) (width 0.2) (layer "B.Cu") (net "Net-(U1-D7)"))
 (segment (start 116.195 65.12) (end 115.11737 66.19763) (width 0.2) (layer "B.Cu") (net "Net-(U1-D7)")))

